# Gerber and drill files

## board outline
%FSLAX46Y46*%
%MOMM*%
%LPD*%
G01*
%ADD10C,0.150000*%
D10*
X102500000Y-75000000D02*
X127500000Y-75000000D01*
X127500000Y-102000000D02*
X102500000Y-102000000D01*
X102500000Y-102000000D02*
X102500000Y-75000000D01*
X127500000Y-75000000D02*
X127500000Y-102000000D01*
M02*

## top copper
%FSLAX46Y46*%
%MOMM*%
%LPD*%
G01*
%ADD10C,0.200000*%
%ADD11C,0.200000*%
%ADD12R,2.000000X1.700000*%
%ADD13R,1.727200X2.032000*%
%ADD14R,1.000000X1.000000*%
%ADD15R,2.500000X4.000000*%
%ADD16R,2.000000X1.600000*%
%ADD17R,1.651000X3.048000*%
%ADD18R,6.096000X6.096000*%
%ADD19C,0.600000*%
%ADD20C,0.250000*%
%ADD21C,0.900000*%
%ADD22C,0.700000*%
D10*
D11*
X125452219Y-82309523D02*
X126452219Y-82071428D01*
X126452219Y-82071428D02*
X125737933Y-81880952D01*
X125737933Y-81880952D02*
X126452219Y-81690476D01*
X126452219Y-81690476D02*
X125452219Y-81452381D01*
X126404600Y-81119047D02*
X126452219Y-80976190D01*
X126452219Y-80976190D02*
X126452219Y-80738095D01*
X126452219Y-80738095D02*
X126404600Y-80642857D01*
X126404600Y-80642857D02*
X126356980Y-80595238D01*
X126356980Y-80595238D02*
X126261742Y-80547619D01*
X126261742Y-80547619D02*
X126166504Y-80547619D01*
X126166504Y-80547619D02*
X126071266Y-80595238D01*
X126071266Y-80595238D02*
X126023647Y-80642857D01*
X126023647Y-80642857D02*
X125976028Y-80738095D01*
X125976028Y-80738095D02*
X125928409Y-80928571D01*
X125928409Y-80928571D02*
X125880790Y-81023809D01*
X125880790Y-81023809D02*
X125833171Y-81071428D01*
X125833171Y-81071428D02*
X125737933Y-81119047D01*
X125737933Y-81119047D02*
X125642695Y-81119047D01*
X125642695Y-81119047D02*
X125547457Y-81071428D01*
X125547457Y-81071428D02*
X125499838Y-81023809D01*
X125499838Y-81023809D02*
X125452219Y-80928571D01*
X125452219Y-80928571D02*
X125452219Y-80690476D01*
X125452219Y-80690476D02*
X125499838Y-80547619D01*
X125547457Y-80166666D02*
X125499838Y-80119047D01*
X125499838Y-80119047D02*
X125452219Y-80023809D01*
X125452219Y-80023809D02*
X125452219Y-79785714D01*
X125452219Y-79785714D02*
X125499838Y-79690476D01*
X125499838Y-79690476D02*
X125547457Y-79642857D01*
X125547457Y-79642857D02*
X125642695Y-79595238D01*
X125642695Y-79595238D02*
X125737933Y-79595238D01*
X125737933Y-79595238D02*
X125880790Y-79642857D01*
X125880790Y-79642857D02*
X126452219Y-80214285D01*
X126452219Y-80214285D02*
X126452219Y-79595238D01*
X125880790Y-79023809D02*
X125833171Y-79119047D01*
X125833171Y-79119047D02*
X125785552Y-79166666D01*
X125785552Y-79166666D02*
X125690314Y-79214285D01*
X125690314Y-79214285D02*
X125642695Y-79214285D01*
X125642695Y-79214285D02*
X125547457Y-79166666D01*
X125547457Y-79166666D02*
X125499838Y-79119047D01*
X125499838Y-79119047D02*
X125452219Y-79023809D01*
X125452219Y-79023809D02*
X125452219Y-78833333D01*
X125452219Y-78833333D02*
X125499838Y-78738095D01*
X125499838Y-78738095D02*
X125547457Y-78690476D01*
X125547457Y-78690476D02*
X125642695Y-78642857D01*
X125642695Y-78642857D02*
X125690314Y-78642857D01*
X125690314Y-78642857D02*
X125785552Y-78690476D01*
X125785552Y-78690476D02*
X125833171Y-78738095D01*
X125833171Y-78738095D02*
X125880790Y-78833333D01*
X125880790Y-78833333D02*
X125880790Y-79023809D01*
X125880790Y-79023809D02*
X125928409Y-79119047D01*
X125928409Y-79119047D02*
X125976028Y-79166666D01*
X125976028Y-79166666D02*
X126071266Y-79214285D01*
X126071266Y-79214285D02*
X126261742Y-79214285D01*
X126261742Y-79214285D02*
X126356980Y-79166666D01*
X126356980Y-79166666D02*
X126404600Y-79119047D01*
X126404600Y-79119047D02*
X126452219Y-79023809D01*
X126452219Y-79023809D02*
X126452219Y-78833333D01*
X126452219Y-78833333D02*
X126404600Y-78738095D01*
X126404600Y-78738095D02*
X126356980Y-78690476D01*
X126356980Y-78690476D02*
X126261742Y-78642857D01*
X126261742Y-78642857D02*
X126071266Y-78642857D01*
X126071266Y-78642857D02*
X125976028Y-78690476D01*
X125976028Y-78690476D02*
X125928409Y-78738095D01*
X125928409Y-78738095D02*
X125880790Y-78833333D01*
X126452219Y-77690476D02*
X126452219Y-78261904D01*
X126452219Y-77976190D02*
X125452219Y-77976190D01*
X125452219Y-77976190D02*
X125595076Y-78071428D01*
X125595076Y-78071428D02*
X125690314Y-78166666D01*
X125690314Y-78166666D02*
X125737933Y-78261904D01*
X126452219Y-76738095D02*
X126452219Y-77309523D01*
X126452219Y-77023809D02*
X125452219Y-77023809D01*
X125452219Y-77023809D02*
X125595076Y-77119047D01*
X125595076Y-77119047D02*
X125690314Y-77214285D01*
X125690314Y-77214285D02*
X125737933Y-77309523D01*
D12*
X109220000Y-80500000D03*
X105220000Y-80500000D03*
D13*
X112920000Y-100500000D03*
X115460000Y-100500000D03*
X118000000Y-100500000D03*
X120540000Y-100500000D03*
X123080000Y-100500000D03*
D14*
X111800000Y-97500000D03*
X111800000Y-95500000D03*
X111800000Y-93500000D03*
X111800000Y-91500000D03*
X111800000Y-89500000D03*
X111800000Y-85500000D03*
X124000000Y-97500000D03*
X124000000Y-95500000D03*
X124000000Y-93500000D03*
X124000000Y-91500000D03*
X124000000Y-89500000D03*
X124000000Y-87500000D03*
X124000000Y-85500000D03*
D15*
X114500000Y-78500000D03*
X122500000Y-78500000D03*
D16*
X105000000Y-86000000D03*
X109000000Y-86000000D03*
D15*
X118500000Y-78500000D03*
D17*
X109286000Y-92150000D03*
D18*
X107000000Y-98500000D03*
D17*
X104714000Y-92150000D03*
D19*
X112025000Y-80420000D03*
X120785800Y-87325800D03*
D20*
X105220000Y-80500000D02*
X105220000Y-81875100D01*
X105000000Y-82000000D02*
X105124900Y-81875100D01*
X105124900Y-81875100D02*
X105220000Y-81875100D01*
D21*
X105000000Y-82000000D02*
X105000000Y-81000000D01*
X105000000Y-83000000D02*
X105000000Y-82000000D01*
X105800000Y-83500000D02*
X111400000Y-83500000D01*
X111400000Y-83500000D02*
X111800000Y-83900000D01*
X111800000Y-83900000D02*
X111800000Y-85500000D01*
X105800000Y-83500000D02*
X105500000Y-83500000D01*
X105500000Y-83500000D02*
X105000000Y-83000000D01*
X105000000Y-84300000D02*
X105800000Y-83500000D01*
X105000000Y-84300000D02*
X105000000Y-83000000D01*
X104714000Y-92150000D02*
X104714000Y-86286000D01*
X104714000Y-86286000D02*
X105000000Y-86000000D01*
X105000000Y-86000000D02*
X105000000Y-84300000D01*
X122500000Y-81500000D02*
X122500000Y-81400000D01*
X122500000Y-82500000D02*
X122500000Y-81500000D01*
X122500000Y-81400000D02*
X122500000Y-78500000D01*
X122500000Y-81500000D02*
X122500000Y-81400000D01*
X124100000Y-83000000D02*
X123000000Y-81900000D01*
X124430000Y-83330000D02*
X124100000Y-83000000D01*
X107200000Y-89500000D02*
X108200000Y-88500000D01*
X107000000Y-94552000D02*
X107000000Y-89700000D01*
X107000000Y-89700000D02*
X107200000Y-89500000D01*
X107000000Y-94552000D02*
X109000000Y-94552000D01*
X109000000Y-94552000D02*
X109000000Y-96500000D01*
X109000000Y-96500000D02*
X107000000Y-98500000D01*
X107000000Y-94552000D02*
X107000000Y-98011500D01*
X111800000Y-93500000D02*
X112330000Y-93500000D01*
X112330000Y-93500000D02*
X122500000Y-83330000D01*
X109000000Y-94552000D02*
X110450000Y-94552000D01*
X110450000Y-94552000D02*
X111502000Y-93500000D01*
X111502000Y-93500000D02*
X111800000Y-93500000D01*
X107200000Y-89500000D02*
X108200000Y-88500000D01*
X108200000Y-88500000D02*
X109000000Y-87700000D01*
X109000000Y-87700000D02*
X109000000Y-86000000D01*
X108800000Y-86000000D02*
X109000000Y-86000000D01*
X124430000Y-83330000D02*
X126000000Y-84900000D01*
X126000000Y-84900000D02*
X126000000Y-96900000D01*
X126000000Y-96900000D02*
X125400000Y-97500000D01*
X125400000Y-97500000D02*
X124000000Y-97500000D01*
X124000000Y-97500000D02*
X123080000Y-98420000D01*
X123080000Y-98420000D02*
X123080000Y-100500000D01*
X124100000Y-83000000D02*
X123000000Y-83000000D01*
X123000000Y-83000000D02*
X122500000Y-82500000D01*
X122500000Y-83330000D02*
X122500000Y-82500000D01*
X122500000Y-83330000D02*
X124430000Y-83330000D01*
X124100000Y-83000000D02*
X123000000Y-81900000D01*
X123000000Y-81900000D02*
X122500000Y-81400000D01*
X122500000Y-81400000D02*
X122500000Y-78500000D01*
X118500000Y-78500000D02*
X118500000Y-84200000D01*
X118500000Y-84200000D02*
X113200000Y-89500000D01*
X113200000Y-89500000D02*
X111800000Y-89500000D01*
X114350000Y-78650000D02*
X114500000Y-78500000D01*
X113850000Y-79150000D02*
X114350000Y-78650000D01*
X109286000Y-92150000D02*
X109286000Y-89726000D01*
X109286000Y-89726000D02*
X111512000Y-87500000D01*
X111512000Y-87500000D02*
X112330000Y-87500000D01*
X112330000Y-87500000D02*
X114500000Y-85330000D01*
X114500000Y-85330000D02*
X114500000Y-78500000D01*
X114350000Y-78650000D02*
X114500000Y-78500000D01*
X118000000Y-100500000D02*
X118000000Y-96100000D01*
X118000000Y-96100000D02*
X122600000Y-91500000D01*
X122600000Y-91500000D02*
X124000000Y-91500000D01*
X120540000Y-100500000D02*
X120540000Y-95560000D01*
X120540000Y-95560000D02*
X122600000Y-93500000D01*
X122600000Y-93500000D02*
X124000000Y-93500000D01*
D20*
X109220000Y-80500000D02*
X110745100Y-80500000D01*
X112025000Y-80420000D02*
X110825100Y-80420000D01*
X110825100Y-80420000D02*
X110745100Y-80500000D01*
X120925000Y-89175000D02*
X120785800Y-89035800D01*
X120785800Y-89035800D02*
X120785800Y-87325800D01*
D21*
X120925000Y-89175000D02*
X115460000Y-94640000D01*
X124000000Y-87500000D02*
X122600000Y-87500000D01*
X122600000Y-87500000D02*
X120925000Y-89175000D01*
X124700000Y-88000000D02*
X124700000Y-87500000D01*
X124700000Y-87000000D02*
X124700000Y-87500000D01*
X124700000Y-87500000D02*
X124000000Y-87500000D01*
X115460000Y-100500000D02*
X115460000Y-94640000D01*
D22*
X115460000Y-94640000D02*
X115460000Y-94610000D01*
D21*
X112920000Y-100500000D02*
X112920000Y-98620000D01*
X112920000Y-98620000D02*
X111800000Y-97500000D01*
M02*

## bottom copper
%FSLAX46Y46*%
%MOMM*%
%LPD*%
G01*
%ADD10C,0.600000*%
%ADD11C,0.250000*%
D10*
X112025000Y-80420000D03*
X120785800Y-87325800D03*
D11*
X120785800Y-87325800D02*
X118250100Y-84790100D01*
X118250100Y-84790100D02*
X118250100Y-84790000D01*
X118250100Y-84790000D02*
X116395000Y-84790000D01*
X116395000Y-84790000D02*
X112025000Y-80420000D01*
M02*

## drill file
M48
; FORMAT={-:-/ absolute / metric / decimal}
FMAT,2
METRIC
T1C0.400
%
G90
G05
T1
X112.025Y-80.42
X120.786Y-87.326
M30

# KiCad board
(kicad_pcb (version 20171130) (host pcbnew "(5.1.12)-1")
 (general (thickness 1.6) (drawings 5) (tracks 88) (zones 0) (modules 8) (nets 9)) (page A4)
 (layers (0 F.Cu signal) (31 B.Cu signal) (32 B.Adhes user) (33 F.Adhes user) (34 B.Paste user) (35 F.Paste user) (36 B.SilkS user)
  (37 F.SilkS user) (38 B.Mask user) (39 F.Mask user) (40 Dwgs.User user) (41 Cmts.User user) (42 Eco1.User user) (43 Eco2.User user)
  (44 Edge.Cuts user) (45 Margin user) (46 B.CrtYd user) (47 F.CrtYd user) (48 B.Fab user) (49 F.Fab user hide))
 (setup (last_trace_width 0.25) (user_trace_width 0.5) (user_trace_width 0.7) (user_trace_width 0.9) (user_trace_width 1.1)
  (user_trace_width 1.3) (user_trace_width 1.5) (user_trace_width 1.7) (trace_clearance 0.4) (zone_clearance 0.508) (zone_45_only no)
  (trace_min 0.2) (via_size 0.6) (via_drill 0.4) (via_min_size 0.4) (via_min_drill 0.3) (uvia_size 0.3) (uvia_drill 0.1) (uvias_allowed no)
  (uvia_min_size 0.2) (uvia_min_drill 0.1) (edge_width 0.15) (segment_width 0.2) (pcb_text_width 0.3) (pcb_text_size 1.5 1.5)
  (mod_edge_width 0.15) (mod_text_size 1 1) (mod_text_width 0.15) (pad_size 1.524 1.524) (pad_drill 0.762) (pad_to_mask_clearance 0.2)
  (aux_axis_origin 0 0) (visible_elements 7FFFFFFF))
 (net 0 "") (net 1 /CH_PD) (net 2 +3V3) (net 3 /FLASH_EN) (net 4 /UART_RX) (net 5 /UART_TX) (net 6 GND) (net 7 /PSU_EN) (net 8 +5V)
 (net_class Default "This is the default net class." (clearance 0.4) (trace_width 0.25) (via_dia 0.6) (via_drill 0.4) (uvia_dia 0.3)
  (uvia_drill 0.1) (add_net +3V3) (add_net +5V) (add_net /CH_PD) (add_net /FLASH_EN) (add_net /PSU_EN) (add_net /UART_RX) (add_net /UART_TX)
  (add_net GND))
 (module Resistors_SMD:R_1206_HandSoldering (layer F.Cu) (at 107.22 80.5 180)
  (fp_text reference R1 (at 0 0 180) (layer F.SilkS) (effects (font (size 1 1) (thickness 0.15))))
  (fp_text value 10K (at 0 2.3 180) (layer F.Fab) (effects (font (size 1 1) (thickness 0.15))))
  (pad 1 smd rect (at -2 0 180) (size 2 1.7) (layers F.Cu F.Paste F.Mask) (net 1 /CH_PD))
  (pad 2 smd rect (at 2 0 180) (size 2 1.7) (layers F.Cu F.Paste F.Mask) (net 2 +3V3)))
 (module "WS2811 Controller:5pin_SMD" (layer F.Cu) (at 112.92 100.5)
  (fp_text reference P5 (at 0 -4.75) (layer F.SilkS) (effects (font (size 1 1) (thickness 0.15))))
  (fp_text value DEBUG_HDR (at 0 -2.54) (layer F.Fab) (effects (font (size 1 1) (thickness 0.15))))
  (pad 1 smd rect (at 0 0) (size 1.7272 2.032) (layers F.Cu F.Paste F.Mask) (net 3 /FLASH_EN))
  (pad 2 smd rect (at 2.54 0) (size 1.7272 2.032) (layers F.Cu F.Paste F.Mask) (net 1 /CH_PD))
  (pad 3 smd rect (at 5.08 0) (size 1.7272 2.032) (layers F.Cu F.Paste F.Mask) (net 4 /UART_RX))
  (pad 4 smd rect (at 7.62 0) (size 1.7272 2.032) (layers F.Cu F.Paste F.Mask) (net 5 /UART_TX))
  (pad 5 smd rect (at 10.16 0) (size 1.7272 2.032) (layers F.Cu F.Paste F.Mask) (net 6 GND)))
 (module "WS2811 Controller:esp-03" (layer F.Cu) (at 117.9 91.6)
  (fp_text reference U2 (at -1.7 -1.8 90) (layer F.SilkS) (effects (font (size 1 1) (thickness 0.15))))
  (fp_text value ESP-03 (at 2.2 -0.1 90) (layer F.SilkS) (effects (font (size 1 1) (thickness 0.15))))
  (pad 14 smd rect (at -6.1 5.9) (size 1 1) (layers F.Cu F.Paste F.Mask) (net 3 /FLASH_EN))
  (pad 13 smd rect (at -6.1 3.9) (size 1 1) (layers F.Cu F.Paste F.Mask))
  (pad 12 smd rect (at -6.1 1.9) (size 1 1) (layers F.Cu F.Paste F.Mask) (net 6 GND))
  (pad 11 smd rect (at -6.1 -0.1) (size 1 1) (layers F.Cu F.Paste F.Mask))
  (pad 10 smd rect (at -6.1 -2.1) (size 1 1) (layers F.Cu F.Paste F.Mask) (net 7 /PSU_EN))
  (pad 8 smd rect (at -6.1 -6.1) (size 1 1) (layers F.Cu F.Paste F.Mask) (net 2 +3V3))
  (pad 1 smd rect (at 6.1 5.9) (size 1 1) (layers F.Cu F.Paste F.Mask) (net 6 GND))
  (pad 2 smd rect (at 6.1 3.9) (size 1 1) (layers F.Cu F.Paste F.Mask))
  (pad 3 smd rect (at 6.1 1.9) (size 1 1) (layers F.Cu F.Paste F.Mask) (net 5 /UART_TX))
  (pad 4 smd rect (at 6.1 -0.1) (size 1 1) (layers F.Cu F.Paste F.Mask) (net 4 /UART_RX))
  (pad 5 smd rect (at 6.1 -2.1) (size 1 1) (layers F.Cu F.Paste F.Mask))
  (pad 6 smd rect (at 6.1 -4.1) (size 1 1) (layers F.Cu F.Paste F.Mask) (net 1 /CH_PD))
  (pad 7 smd rect (at 6.1 -6.1) (size 1 1) (layers F.Cu F.Paste F.Mask)))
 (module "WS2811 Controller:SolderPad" (layer F.Cu) (at 114.5 78.5 270)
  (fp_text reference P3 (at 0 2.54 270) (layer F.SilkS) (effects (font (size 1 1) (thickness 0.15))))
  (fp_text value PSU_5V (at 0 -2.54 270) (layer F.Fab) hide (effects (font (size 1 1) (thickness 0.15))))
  (pad 1 smd rect (at 0 0 270) (size 4 2.5) (layers F.Cu F.Paste F.Mask) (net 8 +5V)))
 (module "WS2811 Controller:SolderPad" (layer F.Cu) (at 122.5 78.5 270)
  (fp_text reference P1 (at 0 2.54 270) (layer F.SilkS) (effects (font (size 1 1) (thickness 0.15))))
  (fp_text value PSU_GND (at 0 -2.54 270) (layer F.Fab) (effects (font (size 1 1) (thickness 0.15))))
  (pad 1 smd rect (at 0 0 270) (size 4 2.5) (layers F.Cu F.Paste F.Mask) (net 6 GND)))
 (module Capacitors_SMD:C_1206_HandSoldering (layer F.Cu) (at 107 86)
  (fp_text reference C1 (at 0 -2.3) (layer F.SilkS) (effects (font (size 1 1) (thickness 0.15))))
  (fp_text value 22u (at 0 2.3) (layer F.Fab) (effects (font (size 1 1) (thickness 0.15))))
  (pad 1 smd rect (at -2 0) (size 2 1.6) (layers F.Cu F.Paste F.Mask) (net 2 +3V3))
  (pad 2 smd rect (at 2 0) (size 2 1.6) (layers F.Cu F.Paste F.Mask) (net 6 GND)))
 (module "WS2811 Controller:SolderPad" (layer F.Cu) (at 118.5 78.5 90)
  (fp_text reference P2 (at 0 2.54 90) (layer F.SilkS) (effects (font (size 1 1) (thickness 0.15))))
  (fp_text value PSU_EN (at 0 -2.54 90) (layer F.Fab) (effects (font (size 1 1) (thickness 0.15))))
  (pad 1 smd rect (at 0 0 90) (size 4 2.5) (layers F.Cu F.Paste F.Mask) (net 7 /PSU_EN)))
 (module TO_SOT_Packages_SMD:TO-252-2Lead (layer F.Cu) (at 107 92.15 180)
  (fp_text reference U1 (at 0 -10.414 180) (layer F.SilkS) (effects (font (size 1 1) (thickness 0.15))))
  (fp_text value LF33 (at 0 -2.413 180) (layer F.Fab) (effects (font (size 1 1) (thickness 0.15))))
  (pad 1 smd rect (at -2.286 0 180) (size 1.651 3.048) (layers F.Cu F.Paste F.Mask) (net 8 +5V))
  (pad 2 smd rect (at 0 -6.35 180) (size 6.096 6.096) (layers F.Cu F.Paste F.Mask) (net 6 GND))
  (pad 3 smd rect (at 2.286 0 180) (size 1.651 3.048) (layers F.Cu F.Paste F.Mask) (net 2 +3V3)))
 (gr_line (start 102.5 75) (end 127.5 75) (layer Edge.Cuts) (width 0.15))
 (gr_line (start 127.5 102) (end 102.5 102) (layer Edge.Cuts) (width 0.15))
 (gr_line (start 102.5 102) (end 102.5 75) (layer Edge.Cuts) (width 0.15))
 (gr_line (start 127.5 75) (end 127.5 102) (layer Edge.Cuts) (width 0.15))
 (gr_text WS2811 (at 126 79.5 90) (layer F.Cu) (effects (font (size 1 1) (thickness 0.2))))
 (segment (start 105.22 80.5) (end 105.22 81.8751) (width 0.25) (layer F.Cu) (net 2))
 (segment (start 105 82) (end 105.1249 81.8751) (width 0.25) (layer F.Cu) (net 2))
 (segment (start 105.1249 81.8751) (end 105.22 81.8751) (width 0.25) (layer F.Cu) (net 2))
 (segment (start 105 82) (end 105 81) (width 0.9) (layer F.Cu) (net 2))
 (segment (start 105 83) (end 105 82) (width 0.9) (layer F.Cu) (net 2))
 (segment (start 105.8 83.5) (end 111.4 83.5) (width 0.9) (layer F.Cu) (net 2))
 (segment (start 111.4 83.5) (end 111.8 83.9) (width 0.9) (layer F.Cu) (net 2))
 (segment (start 111.8 83.9) (end 111.8 85.5) (width 0.9) (layer F.Cu) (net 2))
 (segment (start 105.8 83.5) (end 105.5 83.5) (width 0.9) (layer F.Cu) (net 2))
 (segment (start 105.5 83.5) (end 105 83) (width 0.9) (layer F.Cu) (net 2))
 (segment (start 105 84.3) (end 105.8 83.5) (width 0.9) (layer F.Cu) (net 2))
 (segment (start 105 84.3) (end 105 83) (width 0.9) (layer F.Cu) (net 2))
 (segment (start 104.714 92.15) (end 104.714 86.286) (width 0.9) (layer F.Cu) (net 2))
 (segment (start 104.714 86.286) (end 105 86) (width 0.9) (layer F.Cu) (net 2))
 (segment (start 105 86) (end 105 84.3) (width 0.9) (layer F.Cu) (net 2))
 (segment (start 122.5 81.5) (end 122.5 81.4) (width 0.9) (layer F.Cu) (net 6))
 (segment (start 122.5 82.5) (end 122.5 81.5) (width 0.9) (layer F.Cu) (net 6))
 (segment (start 122.5 81.4) (end 122.5 78.5) (width 0.9) (layer F.Cu) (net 6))
 (segment (start 122.5 81.5) (end 122.5 81.4) (width 0.9) (layer F.Cu) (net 6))
 (segment (start 124.1 83) (end 123 81.9) (width 0.9) (layer F.Cu) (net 6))
 (segment (start 124.43 83.33) (end 124.1 83) (width 0.9) (layer F.Cu) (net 6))
 (segment (start 107.2 89.5) (end 108.2 88.5) (width 0.9) (layer F.Cu) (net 6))
 (segment (start 107 94.552) (end 107 89.7) (width 0.9) (layer F.Cu) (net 6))
 (segment (start 107 89.7) (end 107.2 89.5) (width 0.9) (layer F.Cu) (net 6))
 (segment (start 107 94.552) (end 109 94.552) (width 0.9) (layer F.Cu) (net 6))
 (segment (start 109 94.552) (end 109 96.5) (width 0.9) (layer F.Cu) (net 6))
 (segment (start 109 96.5) (end 107 98.5) (width 0.9) (layer F.Cu) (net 6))
 (segment (start 107 94.552) (end 107 98.0115) (width 0.9) (layer F.Cu) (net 6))
 (segment (start 111.8 93.5) (end 112.33 93.5) (width 0.9) (layer F.Cu) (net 6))
 (segment (start 112.33 93.5) (end 122.5 83.33) (width 0.9) (layer F.Cu) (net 6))
 (segment (start 109 94.552) (end 110.45 94.552) (width 0.9) (layer F.Cu) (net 6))
 (segment (start 110.45 94.552) (end 111.502 93.5) (width 0.9) (layer F.Cu) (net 6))
 (segment (start 111.502 93.5) (end 111.8 93.5) (width 0.9) (layer F.Cu) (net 6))
 (segment (start 107.2 89.5) (end 108.2 88.5) (width 0.9) (layer F.Cu) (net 6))
 (segment (start 108.2 88.5) (end 109 87.7) (width 0.9) (layer F.Cu) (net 6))
 (segment (start 109 87.7) (end 109 86) (width 0.9) (layer F.Cu) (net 6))
 (segment (start 108.8 86) (end 109 86) (width 0.9) (layer F.Cu) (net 6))
 (segment (start 124.43 83.33) (end 126 84.9) (width 0.9) (layer F.Cu) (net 6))
 (segment (start 126 84.9) (end 126 96.9) (width 0.9) (layer F.Cu) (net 6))
 (segment (start 126 96.9) (end 125.4 97.5) (width 0.9) (layer F.Cu) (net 6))
 (segment (start 125.4 97.5) (end 124 97.5) (width 0.9) (layer F.Cu) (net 6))
 (segment (start 124 97.5) (end 123.08 98.42) (width 0.9) (layer F.Cu) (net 6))
 (segment (start 123.08 98.42) (end 123.08 100.5) (width 0.9) (layer F.Cu) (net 6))
 (segment (start 124.1 83) (end 123 83) (width 0.9) (layer F.Cu) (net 6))
 (segment (start 123 83) (end 122.5 82.5) (width 0.9) (layer F.Cu) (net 6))
 (segment (start 122.5 83.33) (end 122.5 82.5) (width 0.9) (layer F.Cu) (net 6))
 (segment (start 122.5 83.33) (end 124.43 83.33) (width 0.9) (layer F.Cu) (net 6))
 (segment (start 124.1 83) (end 123 81.9) (width 0.9) (layer F.Cu) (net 6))
 (segment (start 123 81.9) (end 122.5 81.4) (width 0.9) (layer F.Cu) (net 6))
 (segment (start 122.5 81.4) (end 122.5 78.5) (width 0.9) (layer F.Cu) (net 6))
 (segment (start 118.5 78.5) (end 118.5 84.2) (width 0.9) (layer F.Cu) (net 7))
 (segment (start 118.5 84.2) (end 113.2 89.5) (width 0.9) (layer F.Cu) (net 7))
 (segment (start 113.2 89.5) (end 111.8 89.5) (width 0.9) (layer F.Cu) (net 7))
 (segment (start 114.35 78.65) (end 114.5 78.5) (width 0.9) (layer F.Cu) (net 8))
 (segment (start 113.85 79.15) (end 114.35 78.65) (width 0.9) (layer F.Cu) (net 8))
 (segment (start 109.286 92.15) (end 109.286 89.726) (width 0.9) (layer F.Cu) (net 8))
 (segment (start 109.286 89.726) (end 111.512 87.5) (width 0.9) (layer F.Cu) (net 8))
 (segment (start 111.512 87.5) (end 112.33 87.5) (width 0.9) (layer F.Cu) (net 8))
 (segment (start 112.33 87.5) (end 114.5 85.33) (width 0.9) (layer F.Cu) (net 8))
 (segment (start 114.5 85.33) (end 114.5 78.5) (width 0.9) (layer F.Cu) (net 8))
 (segment (start 114.35 78.65) (end 114.5 78.5) (width 0.9) (layer F.Cu) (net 8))
 (segment (start 118 100.5) (end 118 96.1) (width 0.9) (layer F.Cu) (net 4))
 (segment (start 118 96.1) (end 122.6 91.5) (width 0.9) (layer F.Cu) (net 4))
 (segment (start 122.6 91.5) (end 124 91.5) (width 0.9) (layer F.Cu) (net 4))
 (segment (start 120.54 100.5) (end 120.54 95.56) (width 0.9) (layer F.Cu) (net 5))
 (segment (start 120.54 95.56) (end 122.6 93.5) (width 0.9) (layer F.Cu) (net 5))
 (segment (start 122.6 93.5) (end 124 93.5) (width 0.9) (layer F.Cu) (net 5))
 (segment (start 109.22 80.5) (end 110.7451 80.5) (width 0.25) (layer F.Cu) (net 1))
 (segment (start 112.025 80.42) (end 110.8251 80.42) (width 0.25) (layer F.Cu) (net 1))
 (segment (start 110.8251 80.42) (end 110.7451 80.5) (width 0.25) (layer F.Cu) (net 1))
 (segment (start 120.7858 87.3258) (end 118.2501 84.7901) (width 0.25) (layer B.Cu) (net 1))
 (segment (start 118.2501 84.7901) (end 118.2501 84.79) (width 0.25) (layer B.Cu) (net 1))
 (segment (start 118.2501 84.79) (end 116.395 84.79) (width 0.25) (layer B.Cu) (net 1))
 (segment (start 116.395 84.79) (end 112.025 80.42) (width 0.25) (layer B.Cu) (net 1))
 (segment (start 120.925 89.175) (end 120.7858 89.0358) (width 0.25) (layer F.Cu) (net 1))
 (segment (start 120.7858 89.0358) (end 120.7858 87.3258) (width 0.25) (layer F.Cu) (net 1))
 (segment (start 120.925 89.175) (end 115.46 94.64) (width 0.9) (layer F.Cu) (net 1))
 (segment (start 124 87.5) (end 122.6 87.5) (width 0.9) (layer F.Cu) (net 1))
 (segment (start 122.6 87.5) (end 120.925 89.175) (width 0.9) (layer F.Cu) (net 1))
 (segment (start 124.7 88) (end 124.7 87.5) (width 0.9) (layer F.Cu) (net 1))
 (segment (start 124.7 87) (end 124.7 87.5) (width 0.9) (layer F.Cu) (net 1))
 (segment (start 124.7 87.5) (end 124 87.5) (width 0.9) (layer F.Cu) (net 1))
 (segment (start 115.46 100.5) (end 115.46 94.64) (width 0.9) (layer F.Cu) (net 1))
 (segment (start 115.46 94.64) (end 115.46 94.61) (width 0.7) (layer F.Cu) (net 1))
 (via (at 112.025 80.42) (size 0.6) (layers F.Cu B.Cu) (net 1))
 (via (at 120.7858 87.3258) (size 0.6) (layers F.Cu B.Cu) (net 1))
 (segment (start 112.92 100.5) (end 112.92 98.62) (width 0.9) (layer F.Cu) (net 3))
 (segment (start 112.92 98.62) (end 111.8 97.5) (width 0.9) (layer F.Cu) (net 3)))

